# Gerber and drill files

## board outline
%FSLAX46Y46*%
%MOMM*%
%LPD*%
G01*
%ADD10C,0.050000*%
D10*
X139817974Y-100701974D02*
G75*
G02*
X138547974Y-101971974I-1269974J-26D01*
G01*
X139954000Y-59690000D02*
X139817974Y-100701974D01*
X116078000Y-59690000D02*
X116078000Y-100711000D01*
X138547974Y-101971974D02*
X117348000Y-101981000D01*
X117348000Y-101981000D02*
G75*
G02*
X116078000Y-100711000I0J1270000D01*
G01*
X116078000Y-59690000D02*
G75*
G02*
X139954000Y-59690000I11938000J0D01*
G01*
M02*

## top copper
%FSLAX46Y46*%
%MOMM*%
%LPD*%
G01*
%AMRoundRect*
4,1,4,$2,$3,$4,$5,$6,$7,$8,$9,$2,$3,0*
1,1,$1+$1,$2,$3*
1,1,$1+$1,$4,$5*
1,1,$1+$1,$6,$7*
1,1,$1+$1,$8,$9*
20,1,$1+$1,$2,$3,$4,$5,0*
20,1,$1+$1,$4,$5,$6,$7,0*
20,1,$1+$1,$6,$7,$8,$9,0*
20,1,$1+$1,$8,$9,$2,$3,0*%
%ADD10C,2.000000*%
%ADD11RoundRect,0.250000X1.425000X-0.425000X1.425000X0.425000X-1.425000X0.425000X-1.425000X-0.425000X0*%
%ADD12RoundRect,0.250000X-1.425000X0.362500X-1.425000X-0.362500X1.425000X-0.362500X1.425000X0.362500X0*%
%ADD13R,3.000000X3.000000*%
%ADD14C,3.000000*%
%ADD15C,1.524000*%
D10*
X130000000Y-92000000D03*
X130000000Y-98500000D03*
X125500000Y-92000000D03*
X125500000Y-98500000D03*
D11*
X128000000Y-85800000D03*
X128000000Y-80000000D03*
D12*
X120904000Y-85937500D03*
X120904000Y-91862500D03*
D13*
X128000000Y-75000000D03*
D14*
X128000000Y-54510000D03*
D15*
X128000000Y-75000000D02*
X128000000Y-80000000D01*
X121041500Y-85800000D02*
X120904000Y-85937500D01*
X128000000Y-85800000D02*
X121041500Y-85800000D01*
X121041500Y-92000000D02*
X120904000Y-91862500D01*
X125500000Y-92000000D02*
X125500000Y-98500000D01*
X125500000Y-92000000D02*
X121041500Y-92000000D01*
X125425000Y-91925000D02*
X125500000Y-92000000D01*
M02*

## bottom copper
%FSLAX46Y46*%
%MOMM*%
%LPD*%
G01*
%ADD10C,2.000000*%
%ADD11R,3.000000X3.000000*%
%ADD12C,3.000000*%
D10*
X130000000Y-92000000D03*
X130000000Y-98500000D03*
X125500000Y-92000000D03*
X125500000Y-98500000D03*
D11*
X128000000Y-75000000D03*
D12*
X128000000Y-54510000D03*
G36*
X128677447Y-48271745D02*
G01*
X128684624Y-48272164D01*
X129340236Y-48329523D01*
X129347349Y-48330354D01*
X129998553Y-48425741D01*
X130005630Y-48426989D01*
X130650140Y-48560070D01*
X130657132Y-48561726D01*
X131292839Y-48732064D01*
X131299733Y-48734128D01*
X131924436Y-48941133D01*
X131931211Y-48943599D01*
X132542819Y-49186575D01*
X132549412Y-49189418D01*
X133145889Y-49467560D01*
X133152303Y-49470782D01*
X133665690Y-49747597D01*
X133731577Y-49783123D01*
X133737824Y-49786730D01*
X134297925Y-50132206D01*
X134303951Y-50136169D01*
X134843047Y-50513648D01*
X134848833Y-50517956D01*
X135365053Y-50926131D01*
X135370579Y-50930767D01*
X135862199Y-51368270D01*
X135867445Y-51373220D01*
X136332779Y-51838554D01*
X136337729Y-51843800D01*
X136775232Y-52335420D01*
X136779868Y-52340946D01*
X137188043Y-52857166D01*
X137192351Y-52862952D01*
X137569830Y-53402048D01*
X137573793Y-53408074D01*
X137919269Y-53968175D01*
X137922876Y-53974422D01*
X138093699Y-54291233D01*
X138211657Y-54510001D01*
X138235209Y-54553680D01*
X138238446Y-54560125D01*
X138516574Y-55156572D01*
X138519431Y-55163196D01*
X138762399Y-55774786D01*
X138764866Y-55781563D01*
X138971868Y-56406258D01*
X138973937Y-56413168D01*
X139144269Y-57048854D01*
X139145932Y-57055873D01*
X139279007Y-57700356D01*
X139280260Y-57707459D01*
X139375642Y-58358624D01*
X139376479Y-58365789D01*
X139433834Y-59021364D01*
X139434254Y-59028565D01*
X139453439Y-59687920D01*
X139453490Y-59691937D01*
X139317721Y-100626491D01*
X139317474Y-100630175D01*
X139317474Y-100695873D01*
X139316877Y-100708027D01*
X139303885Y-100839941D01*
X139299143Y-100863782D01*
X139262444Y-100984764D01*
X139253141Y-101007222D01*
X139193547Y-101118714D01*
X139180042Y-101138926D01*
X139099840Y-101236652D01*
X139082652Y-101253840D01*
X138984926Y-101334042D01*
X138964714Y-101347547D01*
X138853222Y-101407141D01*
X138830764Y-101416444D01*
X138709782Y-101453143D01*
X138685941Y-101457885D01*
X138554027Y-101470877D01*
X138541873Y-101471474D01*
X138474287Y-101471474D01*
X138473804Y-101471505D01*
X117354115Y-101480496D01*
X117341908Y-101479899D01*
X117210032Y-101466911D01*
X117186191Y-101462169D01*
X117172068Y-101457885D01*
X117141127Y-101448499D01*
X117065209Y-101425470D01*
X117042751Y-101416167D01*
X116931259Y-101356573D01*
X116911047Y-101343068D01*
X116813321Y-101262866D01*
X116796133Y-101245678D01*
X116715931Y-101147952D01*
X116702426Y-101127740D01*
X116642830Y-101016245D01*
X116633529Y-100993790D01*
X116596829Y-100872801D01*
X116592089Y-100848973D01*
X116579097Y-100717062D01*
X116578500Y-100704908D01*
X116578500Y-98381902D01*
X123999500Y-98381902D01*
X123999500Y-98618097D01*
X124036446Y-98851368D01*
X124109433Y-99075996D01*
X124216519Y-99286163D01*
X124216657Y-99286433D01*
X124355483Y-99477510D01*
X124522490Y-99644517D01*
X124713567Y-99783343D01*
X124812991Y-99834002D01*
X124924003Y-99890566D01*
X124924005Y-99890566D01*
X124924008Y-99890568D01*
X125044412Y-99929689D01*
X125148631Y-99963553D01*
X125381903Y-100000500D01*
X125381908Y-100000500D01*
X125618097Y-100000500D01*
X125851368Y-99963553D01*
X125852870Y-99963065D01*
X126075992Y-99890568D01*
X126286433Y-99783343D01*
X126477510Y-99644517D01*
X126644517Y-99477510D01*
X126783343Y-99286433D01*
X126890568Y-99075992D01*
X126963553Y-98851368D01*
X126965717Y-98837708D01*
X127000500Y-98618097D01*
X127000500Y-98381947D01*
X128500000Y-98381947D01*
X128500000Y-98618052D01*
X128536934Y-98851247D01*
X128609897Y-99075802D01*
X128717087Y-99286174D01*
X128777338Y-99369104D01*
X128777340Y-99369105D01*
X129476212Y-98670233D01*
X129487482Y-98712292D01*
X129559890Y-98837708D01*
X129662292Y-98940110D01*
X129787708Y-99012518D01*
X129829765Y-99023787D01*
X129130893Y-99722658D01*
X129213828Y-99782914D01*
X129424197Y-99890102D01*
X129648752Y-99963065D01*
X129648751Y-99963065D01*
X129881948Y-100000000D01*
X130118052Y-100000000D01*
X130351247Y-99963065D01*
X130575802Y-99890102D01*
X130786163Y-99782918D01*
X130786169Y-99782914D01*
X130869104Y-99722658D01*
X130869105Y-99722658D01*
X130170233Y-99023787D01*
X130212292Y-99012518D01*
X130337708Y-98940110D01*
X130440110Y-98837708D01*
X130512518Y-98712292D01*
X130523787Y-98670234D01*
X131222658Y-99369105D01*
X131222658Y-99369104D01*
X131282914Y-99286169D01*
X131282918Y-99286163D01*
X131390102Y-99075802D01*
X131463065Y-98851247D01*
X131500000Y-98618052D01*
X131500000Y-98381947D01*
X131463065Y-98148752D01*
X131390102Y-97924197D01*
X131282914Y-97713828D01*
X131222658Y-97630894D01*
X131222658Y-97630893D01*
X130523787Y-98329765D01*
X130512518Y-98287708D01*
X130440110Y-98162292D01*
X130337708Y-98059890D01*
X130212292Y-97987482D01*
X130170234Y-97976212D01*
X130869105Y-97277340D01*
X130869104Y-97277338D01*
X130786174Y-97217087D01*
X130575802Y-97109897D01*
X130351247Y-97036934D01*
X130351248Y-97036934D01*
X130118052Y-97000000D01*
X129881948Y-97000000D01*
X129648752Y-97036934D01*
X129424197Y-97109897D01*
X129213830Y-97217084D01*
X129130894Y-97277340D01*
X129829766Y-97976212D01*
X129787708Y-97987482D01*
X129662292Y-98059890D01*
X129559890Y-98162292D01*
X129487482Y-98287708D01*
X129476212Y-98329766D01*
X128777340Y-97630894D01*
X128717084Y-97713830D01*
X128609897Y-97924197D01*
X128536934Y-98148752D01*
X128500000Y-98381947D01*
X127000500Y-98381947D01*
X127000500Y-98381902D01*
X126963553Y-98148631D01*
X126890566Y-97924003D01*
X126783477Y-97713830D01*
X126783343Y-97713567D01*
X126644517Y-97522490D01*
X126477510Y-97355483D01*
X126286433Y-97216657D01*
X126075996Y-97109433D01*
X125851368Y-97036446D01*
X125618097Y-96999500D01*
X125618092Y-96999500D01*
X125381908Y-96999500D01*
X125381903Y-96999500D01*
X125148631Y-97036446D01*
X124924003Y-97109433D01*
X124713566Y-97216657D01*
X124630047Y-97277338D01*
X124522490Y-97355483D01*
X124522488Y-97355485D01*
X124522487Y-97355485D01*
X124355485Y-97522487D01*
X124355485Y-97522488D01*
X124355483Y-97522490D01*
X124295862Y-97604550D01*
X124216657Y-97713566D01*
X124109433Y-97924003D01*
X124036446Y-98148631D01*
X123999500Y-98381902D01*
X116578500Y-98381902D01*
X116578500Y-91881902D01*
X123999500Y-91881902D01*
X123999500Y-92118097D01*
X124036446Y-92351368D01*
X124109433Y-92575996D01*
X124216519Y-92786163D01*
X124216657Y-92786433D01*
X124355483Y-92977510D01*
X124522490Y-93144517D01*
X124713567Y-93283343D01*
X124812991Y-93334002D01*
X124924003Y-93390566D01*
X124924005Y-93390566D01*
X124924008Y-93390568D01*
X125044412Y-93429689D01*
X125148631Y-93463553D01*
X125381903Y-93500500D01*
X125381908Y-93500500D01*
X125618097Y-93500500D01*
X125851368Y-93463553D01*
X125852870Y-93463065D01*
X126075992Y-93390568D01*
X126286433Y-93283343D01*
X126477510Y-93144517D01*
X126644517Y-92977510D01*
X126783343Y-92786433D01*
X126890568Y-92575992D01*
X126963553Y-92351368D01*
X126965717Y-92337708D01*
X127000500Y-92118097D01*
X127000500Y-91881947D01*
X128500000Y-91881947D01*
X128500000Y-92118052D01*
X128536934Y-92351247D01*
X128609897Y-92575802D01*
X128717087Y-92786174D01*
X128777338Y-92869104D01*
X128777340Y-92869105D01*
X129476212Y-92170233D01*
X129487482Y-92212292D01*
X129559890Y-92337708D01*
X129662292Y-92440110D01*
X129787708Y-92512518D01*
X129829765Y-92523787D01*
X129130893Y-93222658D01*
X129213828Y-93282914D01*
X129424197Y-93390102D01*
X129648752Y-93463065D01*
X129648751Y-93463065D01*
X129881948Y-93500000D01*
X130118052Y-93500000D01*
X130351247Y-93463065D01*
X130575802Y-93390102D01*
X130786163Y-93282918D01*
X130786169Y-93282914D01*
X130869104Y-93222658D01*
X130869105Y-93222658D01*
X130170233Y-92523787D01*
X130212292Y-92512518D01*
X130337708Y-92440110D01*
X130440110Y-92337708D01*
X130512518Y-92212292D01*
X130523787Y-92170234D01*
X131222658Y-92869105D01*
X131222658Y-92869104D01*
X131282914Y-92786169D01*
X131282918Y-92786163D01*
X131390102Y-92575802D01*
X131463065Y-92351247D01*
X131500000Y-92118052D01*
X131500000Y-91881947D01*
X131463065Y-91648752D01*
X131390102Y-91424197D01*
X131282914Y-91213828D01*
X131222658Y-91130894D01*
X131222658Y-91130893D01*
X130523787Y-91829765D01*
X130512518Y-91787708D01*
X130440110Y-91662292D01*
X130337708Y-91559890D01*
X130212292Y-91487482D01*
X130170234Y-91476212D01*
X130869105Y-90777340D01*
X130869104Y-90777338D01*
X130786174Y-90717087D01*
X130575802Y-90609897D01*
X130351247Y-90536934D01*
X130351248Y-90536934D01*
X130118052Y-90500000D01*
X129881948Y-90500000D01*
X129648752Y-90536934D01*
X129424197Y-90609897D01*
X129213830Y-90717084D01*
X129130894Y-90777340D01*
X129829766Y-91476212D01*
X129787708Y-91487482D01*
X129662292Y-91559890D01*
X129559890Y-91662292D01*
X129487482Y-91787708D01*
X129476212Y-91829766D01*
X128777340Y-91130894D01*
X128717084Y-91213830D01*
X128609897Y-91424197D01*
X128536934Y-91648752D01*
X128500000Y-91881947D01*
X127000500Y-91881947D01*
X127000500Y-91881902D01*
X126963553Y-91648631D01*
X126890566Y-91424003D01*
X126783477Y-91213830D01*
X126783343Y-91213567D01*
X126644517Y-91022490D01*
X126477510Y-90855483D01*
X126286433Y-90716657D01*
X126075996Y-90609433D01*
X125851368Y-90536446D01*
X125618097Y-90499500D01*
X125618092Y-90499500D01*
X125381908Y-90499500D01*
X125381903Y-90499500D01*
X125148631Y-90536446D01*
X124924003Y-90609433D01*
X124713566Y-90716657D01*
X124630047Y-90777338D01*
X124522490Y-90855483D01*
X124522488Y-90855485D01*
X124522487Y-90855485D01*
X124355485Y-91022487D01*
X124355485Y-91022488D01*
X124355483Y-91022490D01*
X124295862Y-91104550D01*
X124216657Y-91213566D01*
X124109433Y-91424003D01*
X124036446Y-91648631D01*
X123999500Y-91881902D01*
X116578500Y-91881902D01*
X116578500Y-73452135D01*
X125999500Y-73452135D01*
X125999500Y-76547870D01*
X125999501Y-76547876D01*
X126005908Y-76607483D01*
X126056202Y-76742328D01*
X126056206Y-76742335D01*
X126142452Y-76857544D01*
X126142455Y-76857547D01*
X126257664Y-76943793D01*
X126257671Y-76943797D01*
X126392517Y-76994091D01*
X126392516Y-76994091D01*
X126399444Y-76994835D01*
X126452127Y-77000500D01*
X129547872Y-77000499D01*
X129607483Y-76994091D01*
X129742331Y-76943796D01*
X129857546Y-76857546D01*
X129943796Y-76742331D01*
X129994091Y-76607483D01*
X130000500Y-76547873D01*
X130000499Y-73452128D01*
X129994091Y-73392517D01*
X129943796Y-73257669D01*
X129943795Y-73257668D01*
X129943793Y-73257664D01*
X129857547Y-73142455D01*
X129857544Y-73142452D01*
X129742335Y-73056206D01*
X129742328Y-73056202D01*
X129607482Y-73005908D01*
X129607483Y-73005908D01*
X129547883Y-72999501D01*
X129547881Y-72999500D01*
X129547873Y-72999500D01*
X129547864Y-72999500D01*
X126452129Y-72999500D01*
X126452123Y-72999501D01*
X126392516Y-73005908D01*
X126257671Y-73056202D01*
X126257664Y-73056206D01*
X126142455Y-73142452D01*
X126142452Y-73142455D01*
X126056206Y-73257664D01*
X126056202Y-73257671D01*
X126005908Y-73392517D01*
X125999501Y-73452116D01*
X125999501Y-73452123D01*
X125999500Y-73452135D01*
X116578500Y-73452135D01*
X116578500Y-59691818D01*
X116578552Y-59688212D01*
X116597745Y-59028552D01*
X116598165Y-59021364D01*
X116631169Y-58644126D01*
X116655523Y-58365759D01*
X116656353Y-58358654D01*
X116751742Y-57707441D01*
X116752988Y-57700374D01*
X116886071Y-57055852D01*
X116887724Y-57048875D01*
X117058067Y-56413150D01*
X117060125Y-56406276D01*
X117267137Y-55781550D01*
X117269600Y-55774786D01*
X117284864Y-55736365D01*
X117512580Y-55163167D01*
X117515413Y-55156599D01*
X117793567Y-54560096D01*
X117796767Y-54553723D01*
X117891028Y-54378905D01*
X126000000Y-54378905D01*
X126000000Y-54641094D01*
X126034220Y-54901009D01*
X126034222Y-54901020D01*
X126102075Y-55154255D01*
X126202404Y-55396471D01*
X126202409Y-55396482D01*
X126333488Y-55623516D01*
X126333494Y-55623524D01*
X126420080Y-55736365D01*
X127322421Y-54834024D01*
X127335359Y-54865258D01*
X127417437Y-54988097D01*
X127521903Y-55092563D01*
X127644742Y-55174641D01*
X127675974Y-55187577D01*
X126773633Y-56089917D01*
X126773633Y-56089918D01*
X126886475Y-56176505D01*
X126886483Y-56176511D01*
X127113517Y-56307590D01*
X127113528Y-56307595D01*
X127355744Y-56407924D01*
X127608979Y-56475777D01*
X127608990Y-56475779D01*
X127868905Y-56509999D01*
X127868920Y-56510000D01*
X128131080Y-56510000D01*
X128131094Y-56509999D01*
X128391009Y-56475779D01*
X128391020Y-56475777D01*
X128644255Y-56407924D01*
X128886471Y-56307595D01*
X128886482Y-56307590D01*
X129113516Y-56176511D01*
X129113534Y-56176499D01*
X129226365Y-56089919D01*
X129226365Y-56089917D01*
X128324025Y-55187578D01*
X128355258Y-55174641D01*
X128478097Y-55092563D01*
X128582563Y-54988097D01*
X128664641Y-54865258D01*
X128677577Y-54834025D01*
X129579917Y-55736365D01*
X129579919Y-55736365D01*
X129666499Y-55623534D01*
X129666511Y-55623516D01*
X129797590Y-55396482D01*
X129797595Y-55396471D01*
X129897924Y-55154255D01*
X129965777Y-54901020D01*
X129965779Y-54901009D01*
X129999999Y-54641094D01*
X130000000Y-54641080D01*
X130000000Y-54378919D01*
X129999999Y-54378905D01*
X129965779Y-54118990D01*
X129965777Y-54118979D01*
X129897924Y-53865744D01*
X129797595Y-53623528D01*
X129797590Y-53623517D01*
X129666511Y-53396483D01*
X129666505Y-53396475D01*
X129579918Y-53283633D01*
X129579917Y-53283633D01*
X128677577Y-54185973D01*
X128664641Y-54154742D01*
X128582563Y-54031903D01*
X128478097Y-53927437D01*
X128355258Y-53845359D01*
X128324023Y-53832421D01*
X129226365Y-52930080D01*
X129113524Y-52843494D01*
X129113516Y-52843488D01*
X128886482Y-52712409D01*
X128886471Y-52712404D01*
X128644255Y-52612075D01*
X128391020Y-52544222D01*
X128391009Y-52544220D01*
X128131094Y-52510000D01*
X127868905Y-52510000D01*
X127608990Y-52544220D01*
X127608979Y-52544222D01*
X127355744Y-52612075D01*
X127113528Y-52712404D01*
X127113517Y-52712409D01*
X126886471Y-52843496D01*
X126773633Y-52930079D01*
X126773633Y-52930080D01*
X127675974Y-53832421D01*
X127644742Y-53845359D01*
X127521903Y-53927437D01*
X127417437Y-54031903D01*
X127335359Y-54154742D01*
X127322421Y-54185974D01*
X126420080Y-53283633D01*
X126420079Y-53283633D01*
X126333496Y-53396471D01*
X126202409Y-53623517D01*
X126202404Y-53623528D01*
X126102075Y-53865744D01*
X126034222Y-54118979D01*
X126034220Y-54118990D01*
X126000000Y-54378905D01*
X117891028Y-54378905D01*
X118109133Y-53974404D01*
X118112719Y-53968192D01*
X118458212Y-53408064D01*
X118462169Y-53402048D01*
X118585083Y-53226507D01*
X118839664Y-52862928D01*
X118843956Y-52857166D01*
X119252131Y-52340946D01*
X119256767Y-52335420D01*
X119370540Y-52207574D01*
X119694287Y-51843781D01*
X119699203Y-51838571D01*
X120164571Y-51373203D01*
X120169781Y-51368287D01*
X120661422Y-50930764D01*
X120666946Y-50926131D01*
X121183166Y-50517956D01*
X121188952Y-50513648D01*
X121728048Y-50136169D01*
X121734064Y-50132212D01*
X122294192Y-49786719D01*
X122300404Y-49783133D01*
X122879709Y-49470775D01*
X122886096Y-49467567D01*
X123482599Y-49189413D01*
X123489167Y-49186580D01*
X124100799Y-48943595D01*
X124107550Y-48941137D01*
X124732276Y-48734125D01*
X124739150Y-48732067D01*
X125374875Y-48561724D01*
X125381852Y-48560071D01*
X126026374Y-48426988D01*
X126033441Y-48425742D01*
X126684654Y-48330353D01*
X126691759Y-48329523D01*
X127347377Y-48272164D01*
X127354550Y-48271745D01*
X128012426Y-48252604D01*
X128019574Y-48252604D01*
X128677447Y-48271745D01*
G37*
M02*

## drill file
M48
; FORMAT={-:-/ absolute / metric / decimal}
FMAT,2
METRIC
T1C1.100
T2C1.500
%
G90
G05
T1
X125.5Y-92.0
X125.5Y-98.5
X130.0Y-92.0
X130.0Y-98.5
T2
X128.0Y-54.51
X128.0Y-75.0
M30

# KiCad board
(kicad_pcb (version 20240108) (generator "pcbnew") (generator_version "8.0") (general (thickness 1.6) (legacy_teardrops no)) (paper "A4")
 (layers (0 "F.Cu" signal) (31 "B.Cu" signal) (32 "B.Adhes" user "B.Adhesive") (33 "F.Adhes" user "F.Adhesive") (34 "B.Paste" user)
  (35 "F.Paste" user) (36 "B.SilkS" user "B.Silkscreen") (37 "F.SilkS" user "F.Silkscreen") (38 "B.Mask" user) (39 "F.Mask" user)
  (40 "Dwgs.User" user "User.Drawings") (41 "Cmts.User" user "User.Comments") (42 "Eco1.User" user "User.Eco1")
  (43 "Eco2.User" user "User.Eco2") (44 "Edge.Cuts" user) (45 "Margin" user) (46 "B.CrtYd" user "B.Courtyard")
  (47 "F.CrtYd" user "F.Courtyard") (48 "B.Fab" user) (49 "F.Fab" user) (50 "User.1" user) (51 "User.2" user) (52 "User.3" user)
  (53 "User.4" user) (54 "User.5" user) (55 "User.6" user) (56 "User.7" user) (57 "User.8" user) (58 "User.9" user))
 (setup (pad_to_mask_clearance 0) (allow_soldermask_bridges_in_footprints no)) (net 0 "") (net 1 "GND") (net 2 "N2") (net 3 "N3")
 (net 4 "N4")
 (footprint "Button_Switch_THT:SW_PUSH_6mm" (layer "F.Cu") (at 130 92 -90)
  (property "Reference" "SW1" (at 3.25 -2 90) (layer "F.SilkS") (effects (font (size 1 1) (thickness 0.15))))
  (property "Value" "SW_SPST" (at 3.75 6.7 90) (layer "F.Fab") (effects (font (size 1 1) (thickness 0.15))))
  (pad "1" thru_hole circle (at 0 0) (size 2 2) (drill 1.1) (layers "*.Cu" "*.Mask") (remove_unused_layers no) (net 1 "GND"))
  (pad "1" thru_hole circle (at 6.5 0) (size 2 2) (drill 1.1) (layers "*.Cu" "*.Mask") (remove_unused_layers no) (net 1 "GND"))
  (pad "2" thru_hole circle (at 0 4.5) (size 2 2) (drill 1.1) (layers "*.Cu" "*.Mask") (remove_unused_layers no) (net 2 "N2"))
  (pad "2" thru_hole circle (at 6.5 4.5) (size 2 2) (drill 1.1) (layers "*.Cu" "*.Mask") (remove_unused_layers no) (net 2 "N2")))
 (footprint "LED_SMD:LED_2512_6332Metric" (layer "F.Cu") (at 128 82.9 90)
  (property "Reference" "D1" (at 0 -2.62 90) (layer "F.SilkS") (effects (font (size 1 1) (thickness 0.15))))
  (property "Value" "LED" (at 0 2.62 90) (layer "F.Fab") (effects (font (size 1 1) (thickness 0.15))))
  (pad "1" smd roundrect (at -2.9 0 90) (size 1.35 3.35) (layers "F.Cu" "F.Paste" "F.Mask") (roundrect_rratio 0.185185) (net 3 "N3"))
  (pad "2" smd roundrect (at 2.9 0 90) (size 1.35 3.35) (layers "F.Cu" "F.Paste" "F.Mask") (roundrect_rratio 0.185185) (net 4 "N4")))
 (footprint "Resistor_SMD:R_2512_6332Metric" (layer "F.Cu") (at 120.904 88.9 -90)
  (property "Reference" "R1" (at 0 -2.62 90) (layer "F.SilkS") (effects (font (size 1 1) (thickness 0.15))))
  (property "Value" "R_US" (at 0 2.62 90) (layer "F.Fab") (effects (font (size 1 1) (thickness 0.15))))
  (pad "1" smd roundrect (at -2.9625 0 270) (size 1.225 3.35) (layers "F.Cu" "F.Paste" "F.Mask") (roundrect_rratio 0.204082) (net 3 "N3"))
  (pad "2" smd roundrect (at 2.9625 0 270) (size 1.225 3.35) (layers "F.Cu" "F.Paste" "F.Mask") (roundrect_rratio 0.204082) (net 2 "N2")))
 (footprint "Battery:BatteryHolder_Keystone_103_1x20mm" (layer "F.Cu") (at 128 75 90)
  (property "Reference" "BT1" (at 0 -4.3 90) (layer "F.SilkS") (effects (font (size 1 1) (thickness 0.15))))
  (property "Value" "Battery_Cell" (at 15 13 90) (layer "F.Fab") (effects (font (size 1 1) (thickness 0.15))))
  (pad "1" thru_hole rect (at 0 0 90) (size 3 3) (drill 1.5) (layers "*.Cu" "*.Mask") (remove_unused_layers no) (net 4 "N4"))
  (pad "2" thru_hole circle (at 20.49 0 90) (size 3 3) (drill 1.5) (layers "*.Cu" "*.Mask") (remove_unused_layers no) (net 1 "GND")))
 (gr_arc (start 139.817974 100.701974) (mid 139.446 101.6) (end 138.547974 101.971974) (stroke (width 0.05) (type default))
  (layer "Edge.Cuts"))
 (gr_line (start 139.954 59.69) (end 139.817974 100.701974) (stroke (width 0.05) (type default)) (layer "Edge.Cuts"))
 (gr_line (start 116.078 59.69) (end 116.078 100.711) (stroke (width 0.05) (type default)) (layer "Edge.Cuts"))
 (gr_line (start 138.547974 101.971974) (end 117.348 101.981) (stroke (width 0.05) (type default)) (layer "Edge.Cuts"))
 (gr_arc (start 117.348 101.981) (mid 116.449974 101.609026) (end 116.078 100.711) (stroke (width 0.05) (type default)) (layer "Edge.Cuts"))
 (gr_arc (start 116.078 59.69) (mid 128.016 47.752) (end 139.954 59.69) (stroke (width 0.05) (type default)) (layer "Edge.Cuts"))
 (segment (start 128 75) (end 128 80) (width 1.524) (layer "F.Cu") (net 4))
 (segment (start 121.0415 85.8) (end 120.904 85.9375) (width 1.524) (layer "F.Cu") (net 3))
 (segment (start 128 85.8) (end 121.0415 85.8) (width 1.524) (layer "F.Cu") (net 3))
 (segment (start 121.0415 92) (end 120.904 91.8625) (width 1.524) (layer "F.Cu") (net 2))
 (segment (start 125.5 92) (end 125.5 98.5) (width 1.524) (layer "F.Cu") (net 2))
 (segment (start 125.5 92) (end 121.0415 92) (width 1.524) (layer "F.Cu") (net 2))
 (segment (start 125.425 91.925) (end 125.5 92) (width 1.524) (layer "F.Cu") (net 2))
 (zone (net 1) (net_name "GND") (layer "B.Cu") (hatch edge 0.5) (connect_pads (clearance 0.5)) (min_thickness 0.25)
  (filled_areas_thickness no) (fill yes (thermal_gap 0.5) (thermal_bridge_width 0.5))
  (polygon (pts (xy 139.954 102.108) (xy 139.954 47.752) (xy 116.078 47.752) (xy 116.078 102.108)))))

